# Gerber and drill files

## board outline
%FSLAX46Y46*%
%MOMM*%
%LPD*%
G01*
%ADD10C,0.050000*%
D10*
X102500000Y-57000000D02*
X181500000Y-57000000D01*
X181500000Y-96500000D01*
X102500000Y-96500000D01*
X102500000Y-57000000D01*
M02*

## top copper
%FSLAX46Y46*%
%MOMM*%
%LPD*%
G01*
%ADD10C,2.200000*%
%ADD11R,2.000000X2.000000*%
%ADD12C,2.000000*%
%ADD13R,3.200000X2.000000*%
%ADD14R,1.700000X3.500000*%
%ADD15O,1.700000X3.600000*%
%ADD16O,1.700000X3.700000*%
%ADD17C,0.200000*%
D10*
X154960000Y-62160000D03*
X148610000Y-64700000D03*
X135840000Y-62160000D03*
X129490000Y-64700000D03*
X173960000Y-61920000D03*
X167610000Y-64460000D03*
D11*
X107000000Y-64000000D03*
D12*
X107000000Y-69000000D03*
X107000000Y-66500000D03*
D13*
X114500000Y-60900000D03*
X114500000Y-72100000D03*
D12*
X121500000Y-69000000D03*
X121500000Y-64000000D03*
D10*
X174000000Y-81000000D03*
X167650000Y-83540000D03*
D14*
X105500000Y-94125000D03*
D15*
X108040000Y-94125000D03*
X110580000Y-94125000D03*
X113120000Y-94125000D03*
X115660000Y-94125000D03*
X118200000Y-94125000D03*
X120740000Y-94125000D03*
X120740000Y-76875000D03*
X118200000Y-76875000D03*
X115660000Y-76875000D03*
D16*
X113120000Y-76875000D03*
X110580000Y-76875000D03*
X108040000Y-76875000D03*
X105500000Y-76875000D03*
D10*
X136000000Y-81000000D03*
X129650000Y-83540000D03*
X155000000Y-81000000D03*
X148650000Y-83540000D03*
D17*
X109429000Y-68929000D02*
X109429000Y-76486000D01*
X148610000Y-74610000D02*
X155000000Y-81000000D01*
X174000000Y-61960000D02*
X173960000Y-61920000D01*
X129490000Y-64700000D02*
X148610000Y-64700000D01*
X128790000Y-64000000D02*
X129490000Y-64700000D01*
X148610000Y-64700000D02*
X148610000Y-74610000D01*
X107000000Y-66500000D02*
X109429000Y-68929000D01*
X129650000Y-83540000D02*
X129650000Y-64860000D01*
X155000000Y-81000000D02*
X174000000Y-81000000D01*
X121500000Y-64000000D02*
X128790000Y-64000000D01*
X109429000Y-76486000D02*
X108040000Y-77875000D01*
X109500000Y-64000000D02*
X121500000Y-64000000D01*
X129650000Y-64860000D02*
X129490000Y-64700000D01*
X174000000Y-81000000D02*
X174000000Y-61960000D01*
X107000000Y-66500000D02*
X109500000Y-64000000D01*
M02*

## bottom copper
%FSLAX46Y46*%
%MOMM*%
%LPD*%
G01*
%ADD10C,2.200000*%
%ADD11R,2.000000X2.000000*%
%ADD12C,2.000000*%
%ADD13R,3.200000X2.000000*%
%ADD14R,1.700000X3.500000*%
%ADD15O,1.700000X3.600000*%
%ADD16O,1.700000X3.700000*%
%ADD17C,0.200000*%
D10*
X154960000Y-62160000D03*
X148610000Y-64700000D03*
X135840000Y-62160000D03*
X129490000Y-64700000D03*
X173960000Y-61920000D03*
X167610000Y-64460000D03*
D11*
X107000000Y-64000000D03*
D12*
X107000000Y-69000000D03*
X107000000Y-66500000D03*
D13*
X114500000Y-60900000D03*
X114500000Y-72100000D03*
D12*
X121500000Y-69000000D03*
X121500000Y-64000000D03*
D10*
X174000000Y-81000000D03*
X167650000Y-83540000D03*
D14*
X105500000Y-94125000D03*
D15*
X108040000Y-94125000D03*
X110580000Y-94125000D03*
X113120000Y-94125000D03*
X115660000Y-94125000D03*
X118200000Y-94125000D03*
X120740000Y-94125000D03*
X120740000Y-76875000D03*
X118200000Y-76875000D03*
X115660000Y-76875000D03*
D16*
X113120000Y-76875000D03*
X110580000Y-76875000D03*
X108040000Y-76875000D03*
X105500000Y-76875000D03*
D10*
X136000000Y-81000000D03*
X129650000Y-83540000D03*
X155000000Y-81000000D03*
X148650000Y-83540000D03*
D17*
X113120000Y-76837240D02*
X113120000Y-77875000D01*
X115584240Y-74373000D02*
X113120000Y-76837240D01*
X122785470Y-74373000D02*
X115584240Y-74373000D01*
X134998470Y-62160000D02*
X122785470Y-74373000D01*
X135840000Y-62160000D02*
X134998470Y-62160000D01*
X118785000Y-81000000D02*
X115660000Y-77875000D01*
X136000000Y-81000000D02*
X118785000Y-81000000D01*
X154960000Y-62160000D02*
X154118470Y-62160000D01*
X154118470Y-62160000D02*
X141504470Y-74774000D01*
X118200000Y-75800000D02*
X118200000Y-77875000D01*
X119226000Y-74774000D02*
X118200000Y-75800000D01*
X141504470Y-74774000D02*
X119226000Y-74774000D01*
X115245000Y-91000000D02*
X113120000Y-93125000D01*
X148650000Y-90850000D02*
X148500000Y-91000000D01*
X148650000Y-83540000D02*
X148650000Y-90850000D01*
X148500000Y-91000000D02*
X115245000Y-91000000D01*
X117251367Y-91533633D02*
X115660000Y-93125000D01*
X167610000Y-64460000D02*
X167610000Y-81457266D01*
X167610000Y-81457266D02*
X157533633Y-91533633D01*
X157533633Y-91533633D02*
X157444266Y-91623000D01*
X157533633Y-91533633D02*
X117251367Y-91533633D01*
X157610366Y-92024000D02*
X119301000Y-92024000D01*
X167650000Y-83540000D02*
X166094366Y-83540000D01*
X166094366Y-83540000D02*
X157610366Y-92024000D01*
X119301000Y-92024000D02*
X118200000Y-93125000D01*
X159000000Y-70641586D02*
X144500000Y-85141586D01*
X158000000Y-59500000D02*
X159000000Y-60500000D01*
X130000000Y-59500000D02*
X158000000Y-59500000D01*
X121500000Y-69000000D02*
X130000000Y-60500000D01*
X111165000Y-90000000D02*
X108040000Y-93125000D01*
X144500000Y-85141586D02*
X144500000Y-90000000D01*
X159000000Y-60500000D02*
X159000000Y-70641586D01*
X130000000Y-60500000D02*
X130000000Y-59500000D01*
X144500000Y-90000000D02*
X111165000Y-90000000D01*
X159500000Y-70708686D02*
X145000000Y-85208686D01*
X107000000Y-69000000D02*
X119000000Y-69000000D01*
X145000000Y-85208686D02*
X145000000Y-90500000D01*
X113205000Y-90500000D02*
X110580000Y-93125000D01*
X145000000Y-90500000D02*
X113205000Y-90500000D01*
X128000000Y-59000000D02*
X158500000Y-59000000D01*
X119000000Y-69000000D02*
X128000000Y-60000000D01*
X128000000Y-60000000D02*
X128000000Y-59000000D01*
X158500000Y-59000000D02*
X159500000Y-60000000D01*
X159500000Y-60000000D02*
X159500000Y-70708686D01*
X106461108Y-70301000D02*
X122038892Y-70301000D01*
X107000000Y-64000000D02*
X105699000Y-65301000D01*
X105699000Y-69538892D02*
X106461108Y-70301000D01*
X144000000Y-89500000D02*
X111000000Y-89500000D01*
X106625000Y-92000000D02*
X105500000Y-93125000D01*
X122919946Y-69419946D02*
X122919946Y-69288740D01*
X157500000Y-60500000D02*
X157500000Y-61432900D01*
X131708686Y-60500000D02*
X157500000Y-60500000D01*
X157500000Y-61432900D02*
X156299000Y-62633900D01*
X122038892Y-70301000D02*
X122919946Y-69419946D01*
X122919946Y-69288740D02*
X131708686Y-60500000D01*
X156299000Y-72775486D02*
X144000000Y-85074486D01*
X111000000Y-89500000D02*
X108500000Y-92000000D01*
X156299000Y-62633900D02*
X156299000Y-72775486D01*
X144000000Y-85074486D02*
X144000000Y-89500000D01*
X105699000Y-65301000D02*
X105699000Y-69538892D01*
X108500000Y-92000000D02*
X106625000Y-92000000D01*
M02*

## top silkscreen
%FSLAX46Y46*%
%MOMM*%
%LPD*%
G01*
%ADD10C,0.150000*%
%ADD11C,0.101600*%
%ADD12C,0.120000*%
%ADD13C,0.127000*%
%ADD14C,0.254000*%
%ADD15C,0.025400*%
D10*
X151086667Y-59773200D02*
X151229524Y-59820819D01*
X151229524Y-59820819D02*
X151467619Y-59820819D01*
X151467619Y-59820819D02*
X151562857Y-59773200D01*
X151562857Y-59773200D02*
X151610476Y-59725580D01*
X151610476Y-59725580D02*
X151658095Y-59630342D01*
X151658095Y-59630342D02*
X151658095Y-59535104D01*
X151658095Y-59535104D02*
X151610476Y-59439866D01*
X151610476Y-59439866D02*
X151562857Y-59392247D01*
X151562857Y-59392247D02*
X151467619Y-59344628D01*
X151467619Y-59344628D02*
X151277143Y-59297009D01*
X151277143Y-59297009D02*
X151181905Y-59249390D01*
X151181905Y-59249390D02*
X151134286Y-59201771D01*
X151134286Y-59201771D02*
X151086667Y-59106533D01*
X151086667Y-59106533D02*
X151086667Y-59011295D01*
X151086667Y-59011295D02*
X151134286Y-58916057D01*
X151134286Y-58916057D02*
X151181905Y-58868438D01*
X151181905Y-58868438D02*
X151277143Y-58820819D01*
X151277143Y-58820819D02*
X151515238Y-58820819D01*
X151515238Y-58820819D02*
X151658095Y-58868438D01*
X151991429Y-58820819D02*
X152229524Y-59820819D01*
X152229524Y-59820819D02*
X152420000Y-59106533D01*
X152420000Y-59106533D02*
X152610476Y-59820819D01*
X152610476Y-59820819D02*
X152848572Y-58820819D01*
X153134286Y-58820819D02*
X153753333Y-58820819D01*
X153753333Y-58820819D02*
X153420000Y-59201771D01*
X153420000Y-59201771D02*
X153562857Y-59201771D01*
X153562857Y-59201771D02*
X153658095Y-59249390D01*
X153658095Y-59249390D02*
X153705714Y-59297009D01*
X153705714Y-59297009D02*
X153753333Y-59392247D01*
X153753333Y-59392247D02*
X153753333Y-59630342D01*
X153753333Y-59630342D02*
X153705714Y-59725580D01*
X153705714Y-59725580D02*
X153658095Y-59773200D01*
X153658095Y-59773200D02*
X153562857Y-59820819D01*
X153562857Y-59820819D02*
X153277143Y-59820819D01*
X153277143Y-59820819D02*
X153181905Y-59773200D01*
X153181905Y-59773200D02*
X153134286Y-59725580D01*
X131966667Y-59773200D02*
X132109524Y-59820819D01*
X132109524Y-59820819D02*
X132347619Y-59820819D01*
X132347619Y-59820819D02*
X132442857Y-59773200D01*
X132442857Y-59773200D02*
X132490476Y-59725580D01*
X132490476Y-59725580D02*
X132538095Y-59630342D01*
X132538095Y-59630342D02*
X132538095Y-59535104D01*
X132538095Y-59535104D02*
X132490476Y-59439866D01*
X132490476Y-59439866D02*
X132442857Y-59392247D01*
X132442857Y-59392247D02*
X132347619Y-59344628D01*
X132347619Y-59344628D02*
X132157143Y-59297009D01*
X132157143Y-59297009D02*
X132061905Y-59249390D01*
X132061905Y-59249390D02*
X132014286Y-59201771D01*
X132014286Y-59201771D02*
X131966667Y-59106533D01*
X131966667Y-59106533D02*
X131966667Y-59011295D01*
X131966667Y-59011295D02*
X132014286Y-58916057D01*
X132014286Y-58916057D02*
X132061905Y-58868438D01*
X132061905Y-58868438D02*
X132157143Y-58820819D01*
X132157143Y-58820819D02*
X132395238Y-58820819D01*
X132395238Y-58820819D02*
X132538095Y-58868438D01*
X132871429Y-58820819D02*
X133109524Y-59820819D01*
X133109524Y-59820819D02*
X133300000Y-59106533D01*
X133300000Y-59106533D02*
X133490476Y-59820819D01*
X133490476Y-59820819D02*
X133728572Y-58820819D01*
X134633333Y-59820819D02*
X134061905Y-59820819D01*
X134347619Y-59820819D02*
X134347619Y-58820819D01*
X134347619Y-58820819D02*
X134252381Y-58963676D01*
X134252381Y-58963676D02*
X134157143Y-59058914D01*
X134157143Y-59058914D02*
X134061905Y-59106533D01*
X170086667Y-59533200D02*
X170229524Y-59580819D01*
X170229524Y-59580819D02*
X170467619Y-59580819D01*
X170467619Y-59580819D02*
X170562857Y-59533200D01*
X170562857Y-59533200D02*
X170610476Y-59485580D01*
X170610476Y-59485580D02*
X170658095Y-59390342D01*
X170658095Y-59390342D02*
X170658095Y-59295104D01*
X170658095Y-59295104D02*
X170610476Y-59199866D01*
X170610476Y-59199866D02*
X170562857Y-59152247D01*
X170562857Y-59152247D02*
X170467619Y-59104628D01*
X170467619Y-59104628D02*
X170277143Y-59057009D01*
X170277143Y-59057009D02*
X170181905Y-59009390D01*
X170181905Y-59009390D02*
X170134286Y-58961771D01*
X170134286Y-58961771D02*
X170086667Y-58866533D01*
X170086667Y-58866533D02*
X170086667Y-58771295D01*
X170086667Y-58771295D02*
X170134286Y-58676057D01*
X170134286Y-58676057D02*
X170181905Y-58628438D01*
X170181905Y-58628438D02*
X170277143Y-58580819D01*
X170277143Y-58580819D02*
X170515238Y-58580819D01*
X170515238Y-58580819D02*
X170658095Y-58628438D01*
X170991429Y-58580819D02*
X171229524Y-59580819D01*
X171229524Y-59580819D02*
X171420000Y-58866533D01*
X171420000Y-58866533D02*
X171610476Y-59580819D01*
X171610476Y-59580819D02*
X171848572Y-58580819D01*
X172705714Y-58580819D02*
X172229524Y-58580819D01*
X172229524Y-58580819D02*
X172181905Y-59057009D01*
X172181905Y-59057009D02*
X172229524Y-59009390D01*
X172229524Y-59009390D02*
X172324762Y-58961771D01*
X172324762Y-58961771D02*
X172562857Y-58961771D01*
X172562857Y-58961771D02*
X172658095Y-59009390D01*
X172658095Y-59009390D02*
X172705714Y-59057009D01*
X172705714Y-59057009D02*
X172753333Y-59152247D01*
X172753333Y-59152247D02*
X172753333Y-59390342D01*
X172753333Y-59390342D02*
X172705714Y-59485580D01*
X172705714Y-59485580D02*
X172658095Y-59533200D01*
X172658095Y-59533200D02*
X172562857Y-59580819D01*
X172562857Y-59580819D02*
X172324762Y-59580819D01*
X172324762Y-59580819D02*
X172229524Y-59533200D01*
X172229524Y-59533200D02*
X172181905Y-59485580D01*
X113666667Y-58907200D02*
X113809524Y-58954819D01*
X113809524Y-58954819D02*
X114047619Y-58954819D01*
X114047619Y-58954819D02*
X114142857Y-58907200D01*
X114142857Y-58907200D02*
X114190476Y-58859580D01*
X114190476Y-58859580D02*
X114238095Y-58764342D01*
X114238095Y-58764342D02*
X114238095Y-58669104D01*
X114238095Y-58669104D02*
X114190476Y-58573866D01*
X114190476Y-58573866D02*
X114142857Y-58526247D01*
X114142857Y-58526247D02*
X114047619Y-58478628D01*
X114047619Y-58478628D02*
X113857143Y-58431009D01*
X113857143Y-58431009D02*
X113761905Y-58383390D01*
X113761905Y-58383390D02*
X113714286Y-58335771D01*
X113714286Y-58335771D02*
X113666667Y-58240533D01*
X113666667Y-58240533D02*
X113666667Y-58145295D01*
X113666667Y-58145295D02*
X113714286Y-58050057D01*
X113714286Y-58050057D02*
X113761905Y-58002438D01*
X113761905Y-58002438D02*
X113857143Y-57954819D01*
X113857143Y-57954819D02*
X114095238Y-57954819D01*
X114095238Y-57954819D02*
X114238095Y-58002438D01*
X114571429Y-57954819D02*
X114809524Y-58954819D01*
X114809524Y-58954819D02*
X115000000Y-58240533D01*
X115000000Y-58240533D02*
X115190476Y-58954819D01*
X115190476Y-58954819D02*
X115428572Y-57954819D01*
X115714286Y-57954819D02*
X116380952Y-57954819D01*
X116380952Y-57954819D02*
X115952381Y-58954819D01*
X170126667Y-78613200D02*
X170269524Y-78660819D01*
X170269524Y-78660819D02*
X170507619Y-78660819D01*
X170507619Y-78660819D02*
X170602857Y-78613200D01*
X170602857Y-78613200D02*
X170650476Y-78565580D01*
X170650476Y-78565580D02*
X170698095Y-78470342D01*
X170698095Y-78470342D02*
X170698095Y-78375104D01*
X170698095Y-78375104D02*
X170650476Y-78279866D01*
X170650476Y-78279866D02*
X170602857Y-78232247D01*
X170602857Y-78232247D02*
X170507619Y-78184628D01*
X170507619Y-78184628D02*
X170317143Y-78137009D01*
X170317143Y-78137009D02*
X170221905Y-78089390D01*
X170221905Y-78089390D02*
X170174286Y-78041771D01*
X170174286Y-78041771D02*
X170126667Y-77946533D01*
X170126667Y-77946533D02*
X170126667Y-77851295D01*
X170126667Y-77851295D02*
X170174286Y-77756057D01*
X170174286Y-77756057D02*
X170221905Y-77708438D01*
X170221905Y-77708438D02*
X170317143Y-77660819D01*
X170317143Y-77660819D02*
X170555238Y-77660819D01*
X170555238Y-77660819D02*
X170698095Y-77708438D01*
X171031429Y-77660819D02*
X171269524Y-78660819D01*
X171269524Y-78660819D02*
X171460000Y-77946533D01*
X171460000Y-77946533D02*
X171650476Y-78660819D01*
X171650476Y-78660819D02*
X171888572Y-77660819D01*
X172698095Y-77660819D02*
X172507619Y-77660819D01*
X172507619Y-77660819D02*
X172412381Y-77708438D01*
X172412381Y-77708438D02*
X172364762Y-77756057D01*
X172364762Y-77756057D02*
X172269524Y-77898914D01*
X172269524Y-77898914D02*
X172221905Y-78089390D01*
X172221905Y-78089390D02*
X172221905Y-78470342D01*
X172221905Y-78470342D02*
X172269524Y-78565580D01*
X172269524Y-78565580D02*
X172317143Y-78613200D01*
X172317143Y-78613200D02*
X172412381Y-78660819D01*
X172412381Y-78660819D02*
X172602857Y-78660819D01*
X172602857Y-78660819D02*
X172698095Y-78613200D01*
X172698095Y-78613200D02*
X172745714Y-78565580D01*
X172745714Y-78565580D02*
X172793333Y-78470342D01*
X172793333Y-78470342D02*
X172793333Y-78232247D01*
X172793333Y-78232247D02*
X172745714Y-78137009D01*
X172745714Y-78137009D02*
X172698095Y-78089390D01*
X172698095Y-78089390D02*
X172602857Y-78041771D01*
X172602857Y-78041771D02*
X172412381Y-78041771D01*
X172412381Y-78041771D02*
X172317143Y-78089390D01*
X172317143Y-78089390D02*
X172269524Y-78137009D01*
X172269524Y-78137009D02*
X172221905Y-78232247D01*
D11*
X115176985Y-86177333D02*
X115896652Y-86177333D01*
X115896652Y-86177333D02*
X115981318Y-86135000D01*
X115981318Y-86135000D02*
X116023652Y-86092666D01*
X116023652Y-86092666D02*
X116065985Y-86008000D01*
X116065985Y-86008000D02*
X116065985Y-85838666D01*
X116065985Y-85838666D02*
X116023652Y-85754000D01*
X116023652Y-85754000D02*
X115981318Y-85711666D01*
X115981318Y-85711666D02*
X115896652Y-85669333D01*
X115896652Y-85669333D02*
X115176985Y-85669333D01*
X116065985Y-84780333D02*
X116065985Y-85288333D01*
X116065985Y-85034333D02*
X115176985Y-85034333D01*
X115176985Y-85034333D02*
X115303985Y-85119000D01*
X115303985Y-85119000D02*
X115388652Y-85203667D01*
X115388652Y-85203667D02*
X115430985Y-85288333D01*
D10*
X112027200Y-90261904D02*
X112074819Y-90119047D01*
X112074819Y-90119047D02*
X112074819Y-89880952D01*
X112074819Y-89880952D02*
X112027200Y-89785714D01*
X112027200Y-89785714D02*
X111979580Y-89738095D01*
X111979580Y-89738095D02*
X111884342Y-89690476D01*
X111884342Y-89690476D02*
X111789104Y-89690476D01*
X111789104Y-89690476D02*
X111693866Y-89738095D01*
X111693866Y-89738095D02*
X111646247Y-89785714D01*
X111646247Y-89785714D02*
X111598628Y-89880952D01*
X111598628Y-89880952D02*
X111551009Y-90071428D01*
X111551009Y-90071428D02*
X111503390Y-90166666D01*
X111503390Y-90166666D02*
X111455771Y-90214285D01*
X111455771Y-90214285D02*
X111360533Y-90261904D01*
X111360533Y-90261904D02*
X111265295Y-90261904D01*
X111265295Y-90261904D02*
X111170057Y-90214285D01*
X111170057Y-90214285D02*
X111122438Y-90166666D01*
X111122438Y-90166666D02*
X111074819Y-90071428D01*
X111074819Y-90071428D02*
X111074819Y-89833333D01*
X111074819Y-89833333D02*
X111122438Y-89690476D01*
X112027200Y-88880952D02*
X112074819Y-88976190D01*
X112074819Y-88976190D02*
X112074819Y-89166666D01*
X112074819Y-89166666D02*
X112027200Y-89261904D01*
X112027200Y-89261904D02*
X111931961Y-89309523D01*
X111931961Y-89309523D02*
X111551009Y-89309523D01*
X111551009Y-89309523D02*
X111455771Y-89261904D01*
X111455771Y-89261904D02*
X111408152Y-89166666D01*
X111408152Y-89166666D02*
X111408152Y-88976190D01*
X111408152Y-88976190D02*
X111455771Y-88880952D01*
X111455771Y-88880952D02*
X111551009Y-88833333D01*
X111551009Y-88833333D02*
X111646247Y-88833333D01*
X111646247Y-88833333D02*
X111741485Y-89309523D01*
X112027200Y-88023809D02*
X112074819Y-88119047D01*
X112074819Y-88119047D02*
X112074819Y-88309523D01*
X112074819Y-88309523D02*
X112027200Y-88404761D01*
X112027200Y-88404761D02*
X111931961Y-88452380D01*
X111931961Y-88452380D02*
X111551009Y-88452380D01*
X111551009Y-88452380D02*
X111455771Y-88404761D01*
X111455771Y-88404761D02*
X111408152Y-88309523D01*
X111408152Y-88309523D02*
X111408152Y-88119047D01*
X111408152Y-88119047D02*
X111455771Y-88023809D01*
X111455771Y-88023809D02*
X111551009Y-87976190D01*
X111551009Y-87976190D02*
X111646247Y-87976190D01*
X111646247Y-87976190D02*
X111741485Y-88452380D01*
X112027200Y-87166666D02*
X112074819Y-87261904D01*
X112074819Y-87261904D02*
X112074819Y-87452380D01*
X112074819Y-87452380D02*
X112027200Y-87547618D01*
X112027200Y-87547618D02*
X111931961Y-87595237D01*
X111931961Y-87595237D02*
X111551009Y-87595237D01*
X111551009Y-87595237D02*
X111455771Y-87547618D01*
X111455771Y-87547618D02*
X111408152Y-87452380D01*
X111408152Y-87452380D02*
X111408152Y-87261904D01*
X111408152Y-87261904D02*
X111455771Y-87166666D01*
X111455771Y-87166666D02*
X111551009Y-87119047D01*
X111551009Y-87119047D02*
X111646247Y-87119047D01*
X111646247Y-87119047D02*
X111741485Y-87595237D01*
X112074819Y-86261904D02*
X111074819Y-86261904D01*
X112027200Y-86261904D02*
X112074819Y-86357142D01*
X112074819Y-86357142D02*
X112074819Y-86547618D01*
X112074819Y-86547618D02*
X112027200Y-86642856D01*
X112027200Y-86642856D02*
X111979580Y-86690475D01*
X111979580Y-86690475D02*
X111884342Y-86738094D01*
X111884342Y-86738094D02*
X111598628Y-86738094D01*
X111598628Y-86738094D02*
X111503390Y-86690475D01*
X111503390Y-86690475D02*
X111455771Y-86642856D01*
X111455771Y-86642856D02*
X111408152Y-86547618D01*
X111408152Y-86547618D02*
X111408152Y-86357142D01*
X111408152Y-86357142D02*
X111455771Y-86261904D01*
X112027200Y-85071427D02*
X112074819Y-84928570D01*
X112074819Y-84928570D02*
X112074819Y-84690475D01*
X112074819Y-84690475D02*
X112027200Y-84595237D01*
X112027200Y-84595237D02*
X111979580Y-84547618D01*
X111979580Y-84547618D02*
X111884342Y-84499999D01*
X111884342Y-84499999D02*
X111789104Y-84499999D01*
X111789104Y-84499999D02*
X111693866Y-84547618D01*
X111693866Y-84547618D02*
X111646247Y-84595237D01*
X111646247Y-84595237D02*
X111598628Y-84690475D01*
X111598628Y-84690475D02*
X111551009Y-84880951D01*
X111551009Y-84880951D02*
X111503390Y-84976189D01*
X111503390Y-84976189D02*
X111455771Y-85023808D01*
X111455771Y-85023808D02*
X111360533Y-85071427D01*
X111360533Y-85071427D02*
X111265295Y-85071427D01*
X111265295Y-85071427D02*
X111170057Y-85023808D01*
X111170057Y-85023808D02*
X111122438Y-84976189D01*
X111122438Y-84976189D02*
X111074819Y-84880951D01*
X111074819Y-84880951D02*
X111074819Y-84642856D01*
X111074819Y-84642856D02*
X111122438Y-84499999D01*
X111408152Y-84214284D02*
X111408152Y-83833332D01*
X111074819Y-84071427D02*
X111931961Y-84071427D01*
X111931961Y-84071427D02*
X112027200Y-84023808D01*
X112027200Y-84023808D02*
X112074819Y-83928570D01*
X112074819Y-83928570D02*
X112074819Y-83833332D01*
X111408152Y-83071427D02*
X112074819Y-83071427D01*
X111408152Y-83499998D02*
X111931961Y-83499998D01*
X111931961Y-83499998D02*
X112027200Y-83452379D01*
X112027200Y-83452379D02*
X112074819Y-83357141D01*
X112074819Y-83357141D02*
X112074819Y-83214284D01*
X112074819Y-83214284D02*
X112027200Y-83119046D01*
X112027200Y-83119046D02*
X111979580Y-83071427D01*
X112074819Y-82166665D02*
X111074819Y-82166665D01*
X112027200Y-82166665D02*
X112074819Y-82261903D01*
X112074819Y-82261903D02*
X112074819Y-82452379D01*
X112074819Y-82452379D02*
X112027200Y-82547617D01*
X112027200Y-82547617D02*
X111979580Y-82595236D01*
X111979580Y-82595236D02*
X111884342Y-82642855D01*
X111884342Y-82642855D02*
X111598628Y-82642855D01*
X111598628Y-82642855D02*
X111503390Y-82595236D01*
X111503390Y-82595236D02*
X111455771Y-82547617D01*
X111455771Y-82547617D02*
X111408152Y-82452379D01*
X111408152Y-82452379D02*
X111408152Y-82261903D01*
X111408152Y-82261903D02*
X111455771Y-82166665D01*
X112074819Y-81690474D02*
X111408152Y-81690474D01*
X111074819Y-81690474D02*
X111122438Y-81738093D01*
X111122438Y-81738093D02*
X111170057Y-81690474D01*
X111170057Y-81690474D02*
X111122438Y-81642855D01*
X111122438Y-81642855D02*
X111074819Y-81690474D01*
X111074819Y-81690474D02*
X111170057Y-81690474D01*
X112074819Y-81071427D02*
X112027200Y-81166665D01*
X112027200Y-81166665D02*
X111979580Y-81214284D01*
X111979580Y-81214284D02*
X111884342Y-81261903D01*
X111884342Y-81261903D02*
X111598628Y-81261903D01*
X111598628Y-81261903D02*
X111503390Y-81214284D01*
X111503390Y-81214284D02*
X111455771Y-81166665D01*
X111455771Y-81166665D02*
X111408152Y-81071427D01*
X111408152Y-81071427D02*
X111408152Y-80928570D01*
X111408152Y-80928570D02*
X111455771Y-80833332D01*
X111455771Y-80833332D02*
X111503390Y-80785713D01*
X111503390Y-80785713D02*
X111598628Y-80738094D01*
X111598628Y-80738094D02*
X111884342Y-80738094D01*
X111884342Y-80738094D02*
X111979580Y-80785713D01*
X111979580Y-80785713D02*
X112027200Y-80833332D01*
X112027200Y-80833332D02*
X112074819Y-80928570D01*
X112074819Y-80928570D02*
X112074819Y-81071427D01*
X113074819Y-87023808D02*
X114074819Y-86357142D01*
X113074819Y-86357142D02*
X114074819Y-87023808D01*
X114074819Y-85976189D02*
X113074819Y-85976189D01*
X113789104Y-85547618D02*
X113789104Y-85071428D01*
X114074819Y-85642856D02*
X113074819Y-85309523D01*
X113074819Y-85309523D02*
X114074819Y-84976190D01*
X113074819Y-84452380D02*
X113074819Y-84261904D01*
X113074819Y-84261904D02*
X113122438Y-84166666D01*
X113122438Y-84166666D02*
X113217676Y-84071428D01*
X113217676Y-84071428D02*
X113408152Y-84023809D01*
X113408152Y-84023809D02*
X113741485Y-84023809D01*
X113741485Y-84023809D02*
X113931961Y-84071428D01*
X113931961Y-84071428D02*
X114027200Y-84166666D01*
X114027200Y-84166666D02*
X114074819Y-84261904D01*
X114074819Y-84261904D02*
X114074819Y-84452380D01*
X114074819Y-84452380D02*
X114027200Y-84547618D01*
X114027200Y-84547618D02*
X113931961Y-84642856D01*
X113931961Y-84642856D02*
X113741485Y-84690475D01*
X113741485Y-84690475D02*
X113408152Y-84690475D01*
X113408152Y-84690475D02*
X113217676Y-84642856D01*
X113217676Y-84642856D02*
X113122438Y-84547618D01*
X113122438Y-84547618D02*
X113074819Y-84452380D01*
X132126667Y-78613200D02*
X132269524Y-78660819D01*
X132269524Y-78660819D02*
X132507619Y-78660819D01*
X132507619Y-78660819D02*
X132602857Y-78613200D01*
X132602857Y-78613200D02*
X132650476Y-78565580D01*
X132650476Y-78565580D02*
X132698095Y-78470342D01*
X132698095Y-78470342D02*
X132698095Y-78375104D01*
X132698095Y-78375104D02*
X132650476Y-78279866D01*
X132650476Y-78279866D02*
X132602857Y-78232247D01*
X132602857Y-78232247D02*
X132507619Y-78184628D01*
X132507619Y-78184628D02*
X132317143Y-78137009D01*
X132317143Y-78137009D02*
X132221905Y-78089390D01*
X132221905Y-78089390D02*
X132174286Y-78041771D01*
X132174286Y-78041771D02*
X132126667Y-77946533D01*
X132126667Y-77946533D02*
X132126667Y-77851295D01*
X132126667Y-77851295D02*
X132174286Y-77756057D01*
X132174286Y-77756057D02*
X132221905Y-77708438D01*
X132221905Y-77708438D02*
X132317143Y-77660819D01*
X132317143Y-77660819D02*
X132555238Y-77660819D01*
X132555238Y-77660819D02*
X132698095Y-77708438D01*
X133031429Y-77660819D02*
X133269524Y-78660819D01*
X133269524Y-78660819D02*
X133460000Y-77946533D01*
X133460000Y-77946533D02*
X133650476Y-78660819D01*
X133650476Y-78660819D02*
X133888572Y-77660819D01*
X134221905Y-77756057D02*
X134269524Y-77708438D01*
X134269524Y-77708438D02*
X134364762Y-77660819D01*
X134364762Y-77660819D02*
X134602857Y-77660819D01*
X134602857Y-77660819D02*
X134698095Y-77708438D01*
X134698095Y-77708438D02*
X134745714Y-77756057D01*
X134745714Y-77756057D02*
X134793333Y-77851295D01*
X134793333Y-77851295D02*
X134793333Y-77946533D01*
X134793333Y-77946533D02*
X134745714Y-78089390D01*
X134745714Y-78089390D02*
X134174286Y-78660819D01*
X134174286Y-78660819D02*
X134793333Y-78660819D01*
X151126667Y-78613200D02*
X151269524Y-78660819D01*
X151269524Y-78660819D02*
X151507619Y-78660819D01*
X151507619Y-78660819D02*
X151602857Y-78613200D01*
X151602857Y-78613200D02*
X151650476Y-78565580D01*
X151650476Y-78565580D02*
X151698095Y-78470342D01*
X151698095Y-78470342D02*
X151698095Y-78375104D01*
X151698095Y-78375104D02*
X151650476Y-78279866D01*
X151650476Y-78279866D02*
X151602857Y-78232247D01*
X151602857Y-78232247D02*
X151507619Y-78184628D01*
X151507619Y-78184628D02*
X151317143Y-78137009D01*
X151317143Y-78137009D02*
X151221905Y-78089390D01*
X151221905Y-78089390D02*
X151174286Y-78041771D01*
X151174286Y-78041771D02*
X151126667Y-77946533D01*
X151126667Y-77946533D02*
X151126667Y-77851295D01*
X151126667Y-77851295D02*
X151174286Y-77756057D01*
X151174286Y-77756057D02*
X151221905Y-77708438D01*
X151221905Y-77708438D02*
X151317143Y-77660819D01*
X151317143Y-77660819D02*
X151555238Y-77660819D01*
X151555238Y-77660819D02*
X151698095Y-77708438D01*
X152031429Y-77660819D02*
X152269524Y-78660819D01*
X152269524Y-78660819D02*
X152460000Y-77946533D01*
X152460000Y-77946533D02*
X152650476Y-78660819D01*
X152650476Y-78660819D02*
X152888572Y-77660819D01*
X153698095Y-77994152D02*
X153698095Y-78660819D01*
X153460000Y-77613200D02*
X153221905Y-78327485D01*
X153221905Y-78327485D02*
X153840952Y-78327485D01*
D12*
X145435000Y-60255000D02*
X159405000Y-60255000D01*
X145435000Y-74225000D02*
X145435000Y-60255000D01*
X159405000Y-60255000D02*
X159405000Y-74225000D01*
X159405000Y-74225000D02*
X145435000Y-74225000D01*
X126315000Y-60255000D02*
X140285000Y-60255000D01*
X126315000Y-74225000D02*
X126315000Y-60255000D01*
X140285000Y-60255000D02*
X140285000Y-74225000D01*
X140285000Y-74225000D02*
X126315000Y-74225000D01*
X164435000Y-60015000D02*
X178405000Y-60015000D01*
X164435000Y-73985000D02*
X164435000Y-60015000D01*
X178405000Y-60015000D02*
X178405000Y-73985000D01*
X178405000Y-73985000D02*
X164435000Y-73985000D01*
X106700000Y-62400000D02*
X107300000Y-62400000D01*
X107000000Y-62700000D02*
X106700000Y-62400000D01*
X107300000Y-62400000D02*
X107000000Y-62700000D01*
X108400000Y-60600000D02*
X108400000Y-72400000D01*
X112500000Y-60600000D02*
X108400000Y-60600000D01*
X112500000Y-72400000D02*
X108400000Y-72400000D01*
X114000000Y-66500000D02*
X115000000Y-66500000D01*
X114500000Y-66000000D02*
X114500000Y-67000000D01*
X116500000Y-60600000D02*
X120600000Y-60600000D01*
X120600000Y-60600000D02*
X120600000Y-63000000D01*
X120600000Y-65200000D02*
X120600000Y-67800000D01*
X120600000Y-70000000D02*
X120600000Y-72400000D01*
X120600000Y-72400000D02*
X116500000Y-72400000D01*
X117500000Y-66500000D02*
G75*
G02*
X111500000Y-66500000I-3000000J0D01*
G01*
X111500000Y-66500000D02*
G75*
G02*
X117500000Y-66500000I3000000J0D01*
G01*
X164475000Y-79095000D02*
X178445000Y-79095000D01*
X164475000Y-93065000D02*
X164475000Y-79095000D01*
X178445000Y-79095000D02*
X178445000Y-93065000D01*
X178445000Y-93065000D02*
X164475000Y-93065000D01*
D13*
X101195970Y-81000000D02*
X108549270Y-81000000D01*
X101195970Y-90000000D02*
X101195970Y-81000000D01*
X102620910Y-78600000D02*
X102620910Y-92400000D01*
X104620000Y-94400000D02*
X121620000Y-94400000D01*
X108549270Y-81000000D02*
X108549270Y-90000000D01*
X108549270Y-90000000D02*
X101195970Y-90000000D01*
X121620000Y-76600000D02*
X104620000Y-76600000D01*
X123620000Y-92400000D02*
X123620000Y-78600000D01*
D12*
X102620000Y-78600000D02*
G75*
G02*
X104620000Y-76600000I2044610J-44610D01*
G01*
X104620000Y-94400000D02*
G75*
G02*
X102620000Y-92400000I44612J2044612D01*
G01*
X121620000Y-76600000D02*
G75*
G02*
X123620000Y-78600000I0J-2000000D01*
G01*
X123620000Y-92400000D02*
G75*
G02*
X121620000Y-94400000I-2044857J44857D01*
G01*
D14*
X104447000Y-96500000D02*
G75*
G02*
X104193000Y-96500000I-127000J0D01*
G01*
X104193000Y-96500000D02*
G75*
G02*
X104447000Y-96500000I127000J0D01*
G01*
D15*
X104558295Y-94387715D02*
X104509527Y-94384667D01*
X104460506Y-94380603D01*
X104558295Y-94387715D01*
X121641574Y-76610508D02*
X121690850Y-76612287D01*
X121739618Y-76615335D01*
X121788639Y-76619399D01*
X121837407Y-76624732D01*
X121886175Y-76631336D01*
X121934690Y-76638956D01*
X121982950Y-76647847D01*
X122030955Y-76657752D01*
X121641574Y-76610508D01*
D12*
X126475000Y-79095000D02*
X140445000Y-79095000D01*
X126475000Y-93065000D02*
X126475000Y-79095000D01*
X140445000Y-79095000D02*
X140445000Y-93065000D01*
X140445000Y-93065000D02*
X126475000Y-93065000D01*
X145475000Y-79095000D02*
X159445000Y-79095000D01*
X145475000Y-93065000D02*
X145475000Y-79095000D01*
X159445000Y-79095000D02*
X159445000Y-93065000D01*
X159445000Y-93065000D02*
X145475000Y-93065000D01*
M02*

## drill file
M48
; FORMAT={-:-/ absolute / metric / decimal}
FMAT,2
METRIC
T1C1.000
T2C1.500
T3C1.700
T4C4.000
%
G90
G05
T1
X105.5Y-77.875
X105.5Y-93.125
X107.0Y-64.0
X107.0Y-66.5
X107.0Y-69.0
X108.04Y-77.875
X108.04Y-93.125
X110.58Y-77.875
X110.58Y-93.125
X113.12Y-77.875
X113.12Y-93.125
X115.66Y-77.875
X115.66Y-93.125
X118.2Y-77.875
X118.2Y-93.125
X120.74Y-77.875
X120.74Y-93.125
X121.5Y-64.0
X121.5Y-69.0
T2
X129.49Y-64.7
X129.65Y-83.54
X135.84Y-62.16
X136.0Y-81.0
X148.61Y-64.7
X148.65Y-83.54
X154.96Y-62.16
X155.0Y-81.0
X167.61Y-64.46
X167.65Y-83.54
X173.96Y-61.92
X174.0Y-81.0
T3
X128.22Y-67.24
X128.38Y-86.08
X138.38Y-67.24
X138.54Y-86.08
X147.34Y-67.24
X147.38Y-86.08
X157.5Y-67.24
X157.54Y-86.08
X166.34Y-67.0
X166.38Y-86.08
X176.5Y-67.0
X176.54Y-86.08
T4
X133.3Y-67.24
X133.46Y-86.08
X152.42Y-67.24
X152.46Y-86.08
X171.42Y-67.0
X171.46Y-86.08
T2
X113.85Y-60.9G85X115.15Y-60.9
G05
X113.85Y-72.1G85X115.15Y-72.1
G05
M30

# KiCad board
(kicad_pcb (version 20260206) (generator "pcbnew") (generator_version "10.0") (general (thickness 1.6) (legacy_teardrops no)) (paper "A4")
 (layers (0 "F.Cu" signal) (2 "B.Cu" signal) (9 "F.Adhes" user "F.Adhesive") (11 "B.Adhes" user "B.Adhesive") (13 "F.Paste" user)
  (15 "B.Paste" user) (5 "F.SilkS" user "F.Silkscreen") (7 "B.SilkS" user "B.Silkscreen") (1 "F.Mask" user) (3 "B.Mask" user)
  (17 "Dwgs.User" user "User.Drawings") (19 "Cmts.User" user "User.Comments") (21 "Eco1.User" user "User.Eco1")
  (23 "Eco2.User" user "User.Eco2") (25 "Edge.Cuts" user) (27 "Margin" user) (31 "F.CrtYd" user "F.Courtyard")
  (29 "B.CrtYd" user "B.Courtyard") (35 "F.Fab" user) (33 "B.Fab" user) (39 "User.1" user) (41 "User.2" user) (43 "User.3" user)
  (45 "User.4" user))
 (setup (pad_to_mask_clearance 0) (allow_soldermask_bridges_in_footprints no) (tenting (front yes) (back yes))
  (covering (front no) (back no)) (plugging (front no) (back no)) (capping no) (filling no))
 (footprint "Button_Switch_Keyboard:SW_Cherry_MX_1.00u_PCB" (layer "F.Cu") (at 154.96 62.16)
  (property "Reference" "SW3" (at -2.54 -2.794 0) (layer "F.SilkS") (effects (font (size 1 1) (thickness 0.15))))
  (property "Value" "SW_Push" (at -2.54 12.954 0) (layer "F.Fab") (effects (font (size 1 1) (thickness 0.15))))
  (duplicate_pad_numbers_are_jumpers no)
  (fp_line (start -9.525 -1.905) (end 4.445 -1.905) (stroke (width 0.12) (type solid)) (layer "F.SilkS"))
  (fp_line (start -9.525 12.065) (end -9.525 -1.905) (stroke (width 0.12) (type solid)) (layer "F.SilkS"))
  (fp_line (start 4.445 -1.905) (end 4.445 12.065) (stroke (width 0.12) (type solid)) (layer "F.SilkS"))
  (fp_line (start 4.445 12.065) (end -9.525 12.065) (stroke (width 0.12) (type solid)) (layer "F.SilkS"))
  (pad "" np_thru_hole circle (at -7.62 5.08) (size 1.7 1.7) (drill 1.7) (layers "*.Cu" "*.Mask"))
  (pad "" np_thru_hole circle (at -2.54 5.08) (size 4 4) (drill 4) (layers "*.Cu" "*.Mask"))
  (pad "" np_thru_hole circle (at 2.54 5.08) (size 1.7 1.7) (drill 1.7) (layers "*.Cu" "*.Mask"))
  (pad "1" thru_hole circle (at 0 0) (size 2.2 2.2) (drill 1.5) (layers "*.Cu" "*.Mask") (remove_unused_layers no)
   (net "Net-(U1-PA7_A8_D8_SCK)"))
  (pad "2" thru_hole circle (at -6.35 2.54) (size 2.2 2.2) (drill 1.5) (layers "*.Cu" "*.Mask") (remove_unused_layers no) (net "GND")))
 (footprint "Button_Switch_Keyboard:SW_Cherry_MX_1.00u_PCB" (layer "F.Cu") (at 135.84 62.16)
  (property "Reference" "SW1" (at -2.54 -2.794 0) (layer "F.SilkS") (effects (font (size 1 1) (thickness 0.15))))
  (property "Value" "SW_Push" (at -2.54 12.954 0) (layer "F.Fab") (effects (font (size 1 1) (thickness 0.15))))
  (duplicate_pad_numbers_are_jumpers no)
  (fp_line (start -9.525 -1.905) (end 4.445 -1.905) (stroke (width 0.12) (type solid)) (layer "F.SilkS"))
  (fp_line (start -9.525 12.065) (end -9.525 -1.905) (stroke (width 0.12) (type solid)) (layer "F.SilkS"))
  (fp_line (start 4.445 -1.905) (end 4.445 12.065) (stroke (width 0.12) (type solid)) (layer "F.SilkS"))
  (fp_line (start 4.445 12.065) (end -9.525 12.065) (stroke (width 0.12) (type solid)) (layer "F.SilkS"))
  (pad "" np_thru_hole circle (at -7.62 5.08) (size 1.7 1.7) (drill 1.7) (layers "*.Cu" "*.Mask"))
  (pad "" np_thru_hole circle (at -2.54 5.08) (size 4 4) (drill 4) (layers "*.Cu" "*.Mask"))
  (pad "" np_thru_hole circle (at 2.54 5.08) (size 1.7 1.7) (drill 1.7) (layers "*.Cu" "*.Mask"))
  (pad "1" thru_hole circle (at 0 0) (size 2.2 2.2) (drill 1.5) (layers "*.Cu" "*.Mask") (remove_unused_layers no)
   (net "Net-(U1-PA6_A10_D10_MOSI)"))
  (pad "2" thru_hole circle (at -6.35 2.54) (size 2.2 2.2) (drill 1.5) (layers "*.Cu" "*.Mask") (remove_unused_layers no) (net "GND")))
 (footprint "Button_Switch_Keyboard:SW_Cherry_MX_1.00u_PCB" (layer "F.Cu") (at 173.96 61.92)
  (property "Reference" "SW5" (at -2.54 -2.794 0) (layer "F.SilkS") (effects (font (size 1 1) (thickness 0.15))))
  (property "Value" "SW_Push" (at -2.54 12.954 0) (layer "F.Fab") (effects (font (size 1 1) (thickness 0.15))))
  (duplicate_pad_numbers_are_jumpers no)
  (fp_line (start -9.525 -1.905) (end 4.445 -1.905) (stroke (width 0.12) (type solid)) (layer "F.SilkS"))
  (fp_line (start -9.525 12.065) (end -9.525 -1.905) (stroke (width 0.12) (type solid)) (layer "F.SilkS"))
  (fp_line (start 4.445 -1.905) (end 4.445 12.065) (stroke (width 0.12) (type solid)) (layer "F.SilkS"))
  (fp_line (start 4.445 12.065) (end -9.525 12.065) (stroke (width 0.12) (type solid)) (layer "F.SilkS"))
  (pad "" np_thru_hole circle (at -7.62 5.08) (size 1.7 1.7) (drill 1.7) (layers "*.Cu" "*.Mask"))
  (pad "" np_thru_hole circle (at -2.54 5.08) (size 4 4) (drill 4) (layers "*.Cu" "*.Mask"))
  (pad "" np_thru_hole circle (at 2.54 5.08) (size 1.7 1.7) (drill 1.7) (layers "*.Cu" "*.Mask"))
  (pad "1" thru_hole circle (at 0 0) (size 2.2 2.2) (drill 1.5) (layers "*.Cu" "*.Mask") (remove_unused_layers no) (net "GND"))
  (pad "2" thru_hole circle (at -6.35 2.54) (size 2.2 2.2) (drill 1.5) (layers "*.Cu" "*.Mask") (remove_unused_layers no)
   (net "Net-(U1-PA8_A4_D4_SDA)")))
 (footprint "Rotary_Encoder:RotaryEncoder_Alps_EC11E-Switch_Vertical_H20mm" (layer "F.Cu") (at 107 64)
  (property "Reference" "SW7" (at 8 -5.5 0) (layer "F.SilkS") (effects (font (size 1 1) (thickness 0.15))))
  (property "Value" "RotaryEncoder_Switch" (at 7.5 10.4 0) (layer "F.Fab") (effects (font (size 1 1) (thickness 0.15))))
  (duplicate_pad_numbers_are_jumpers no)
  (fp_line (start -0.3 -1.6) (end 0.3 -1.6) (stroke (width 0.12) (type solid)) (layer "F.SilkS"))
  (fp_line (start 0 -1.3) (end -0.3 -1.6) (stroke (width 0.12) (type solid)) (layer "F.SilkS"))
  (fp_line (start 0.3 -1.6) (end 0 -1.3) (stroke (width 0.12) (type solid)) (layer "F.SilkS"))
  (fp_line (start 1.4 -3.4) (end 1.4 8.4) (stroke (width 0.12) (type solid)) (layer "F.SilkS"))
  (fp_line (start 5.5 -3.4) (end 1.4 -3.4) (stroke (width 0.12) (type solid)) (layer "F.SilkS"))
  (fp_line (start 5.5 8.4) (end 1.4 8.4) (stroke (width 0.12) (type solid)) (layer "F.SilkS"))
  (fp_line (start 7 2.5) (end 8 2.5) (stroke (width 0.12) (type solid)) (layer "F.SilkS"))
  (fp_line (start 7.5 2) (end 7.5 3) (stroke (width 0.12) (type solid)) (layer "F.SilkS"))
  (fp_line (start 9.5 -3.4) (end 13.6 -3.4) (stroke (width 0.12) (type solid)) (layer "F.SilkS"))
  (fp_line (start 13.6 -3.4) (end 13.6 -1) (stroke (width 0.12) (type solid)) (layer "F.SilkS"))
  (fp_line (start 13.6 1.2) (end 13.6 3.8) (stroke (width 0.12) (type solid)) (layer "F.SilkS"))
  (fp_line (start 13.6 6) (end 13.6 8.4) (stroke (width 0.12) (type solid)) (layer "F.SilkS"))
  (fp_line (start 13.6 8.4) (end 9.5 8.4) (stroke (width 0.12) (type solid)) (layer "F.SilkS"))
  (fp_circle (center 7.5 2.5) (end 10.5 2.5) (stroke (width 0.12) (type solid)) (fill no) (layer "F.SilkS"))
  (pad "A" thru_hole rect (at 0 0) (size 2 2) (drill 1) (layers "*.Cu" "*.Mask") (remove_unused_layers no) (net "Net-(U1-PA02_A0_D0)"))
  (pad "B" thru_hole circle (at 0 5) (size 2 2) (drill 1) (layers "*.Cu" "*.Mask") (remove_unused_layers no) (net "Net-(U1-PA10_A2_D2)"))
  (pad "C" thru_hole circle (at 0 2.5) (size 2 2) (drill 1) (layers "*.Cu" "*.Mask") (remove_unused_layers no) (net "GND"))
  (pad "MP" thru_hole rect (at 7.5 -3.1) (size 3.2 2) (drill oval 2.8 1.5) (layers "*.Cu" "*.Mask") (remove_unused_layers no))
  (pad "MP" thru_hole rect (at 7.5 8.1) (size 3.2 2) (drill oval 2.8 1.5) (layers "*.Cu" "*.Mask") (remove_unused_layers no))
  (pad "S1" thru_hole circle (at 14.5 5) (size 2 2) (drill 1) (layers "*.Cu" "*.Mask") (remove_unused_layers no) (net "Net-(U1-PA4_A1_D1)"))
  (pad "S2" thru_hole circle (at 14.5 0) (size 2 2) (drill 1) (layers "*.Cu" "*.Mask") (remove_unused_layers no) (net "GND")))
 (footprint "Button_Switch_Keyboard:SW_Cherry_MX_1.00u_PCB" (layer "F.Cu") (at 174 81)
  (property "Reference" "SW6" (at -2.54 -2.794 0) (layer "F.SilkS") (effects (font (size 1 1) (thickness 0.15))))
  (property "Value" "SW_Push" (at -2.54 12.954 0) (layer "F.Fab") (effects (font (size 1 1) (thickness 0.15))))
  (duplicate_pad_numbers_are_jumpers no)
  (fp_line (start -9.525 -1.905) (end 4.445 -1.905) (stroke (width 0.12) (type solid)) (layer "F.SilkS"))
  (fp_line (start -9.525 12.065) (end -9.525 -1.905) (stroke (width 0.12) (type solid)) (layer "F.SilkS"))
  (fp_line (start 4.445 -1.905) (end 4.445 12.065) (stroke (width 0.12) (type solid)) (layer "F.SilkS"))
  (fp_line (start 4.445 12.065) (end -9.525 12.065) (stroke (width 0.12) (type solid)) (layer "F.SilkS"))
  (pad "" np_thru_hole circle (at -7.62 5.08) (size 1.7 1.7) (drill 1.7) (layers "*.Cu" "*.Mask"))
  (pad "" np_thru_hole circle (at -2.54 5.08) (size 4 4) (drill 4) (layers "*.Cu" "*.Mask"))
  (pad "" np_thru_hole circle (at 2.54 5.08) (size 1.7 1.7) (drill 1.7) (layers "*.Cu" "*.Mask"))
  (pad "1" thru_hole circle (at 0 0) (size 2.2 2.2) (drill 1.5) (layers "*.Cu" "*.Mask") (remove_unused_layers no) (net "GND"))
  (pad "2" thru_hole circle (at -6.35 2.54) (size 2.2 2.2) (drill 1.5) (layers "*.Cu" "*.Mask") (remove_unused_layers no)
   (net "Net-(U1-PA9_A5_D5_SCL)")))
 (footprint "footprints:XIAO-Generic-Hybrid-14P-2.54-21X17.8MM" (layer "F.Cu") (at 113.12 85.5 90)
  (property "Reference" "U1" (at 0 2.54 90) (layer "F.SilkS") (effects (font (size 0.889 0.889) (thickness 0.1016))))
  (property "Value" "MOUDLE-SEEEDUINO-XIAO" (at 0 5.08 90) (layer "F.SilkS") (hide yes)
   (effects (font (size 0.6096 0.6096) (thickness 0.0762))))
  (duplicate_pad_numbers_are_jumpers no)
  (fp_line (start 4.5 -11.92403) (end 4.5 -4.57073) (stroke (width 0.127) (type solid)) (layer "F.SilkS"))
  (fp_line (start -4.5 -11.92403) (end 4.5 -11.92403) (stroke (width 0.127) (type solid)) (layer "F.SilkS"))
  (fp_line (start 6.9 -10.49909) (end -6.9 -10.49909) (stroke (width 0.127) (type solid)) (layer "F.SilkS"))
  (fp_line (start -8.9 -8.5) (end -8.9 8.5) (stroke (width 0.127) (type solid)) (layer "F.SilkS"))
  (fp_line (start 4.5 -4.57073) (end -4.5 -4.57073) (stroke (width 0.127) (type solid)) (layer "F.SilkS"))
  (fp_line (start -4.5 -4.57073) (end -4.5 -11.92403) (stroke (width 0.127) (type solid)) (layer "F.SilkS"))
  (fp_line (start 8.9 8.5) (end 8.9 -8.5) (stroke (width 0.127) (type solid)) (layer "F.SilkS"))
  (fp_line (start -6.9 10.5) (end 6.9 10.5) (stroke (width 0.127) (type solid)) (layer "F.SilkS"))
  (fp_arc (start 6.9 -10.5) (mid 8.301491 -9.901491) (end 8.9 -8.5) (stroke (width 0.12) (type solid)) (layer "F.SilkS"))
  (fp_arc (start -8.9 -8.5) (mid -8.301491 -9.901491) (end -6.9 -10.5) (stroke (width 0.12) (type solid)) (layer "F.SilkS"))
  (fp_arc (start 8.9 8.5) (mid 8.314214 9.914214) (end 6.9 10.5) (stroke (width 0.12) (type solid)) (layer "F.SilkS"))
  (fp_arc (start -6.9 10.5) (mid -8.301423 9.901423) (end -8.9 8.5) (stroke (width 0.12) (type solid)) (layer "F.SilkS"))
  (fp_circle (center -11 -8.8) (end -11 -9.054) (stroke (width 0) (type solid)) (fill yes) (layer "F.SilkS"))
  (fp_poly
   (pts (xy -8.887715 -8.561705) (xy -8.884667 -8.610473) (xy -8.880603 -8.659494)) (stroke (width 0.0254) (type solid)) (fill no)
   (layer "F.SilkS"))
  (fp_poly
   (pts (xy 8.889492 8.521574) (xy 8.887713 8.57085) (xy 8.884665 8.619618) (xy 8.880601 8.668639) (xy 8.875268 8.717407)
    (xy 8.868664 8.766175) (xy 8.861044 8.81469) (xy 8.852153 8.86295) (xy 8.842248 8.910955))
   (stroke (width 0.0254) (type solid)) (fill no) (layer "F.SilkS"))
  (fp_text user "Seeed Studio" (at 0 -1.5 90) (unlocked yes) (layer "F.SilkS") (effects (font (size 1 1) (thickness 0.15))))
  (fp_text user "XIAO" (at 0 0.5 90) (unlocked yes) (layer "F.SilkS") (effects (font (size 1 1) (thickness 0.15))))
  (pad "1" thru_hole rect (at -7.625 -7.62 90) (size 3.5 1.7) (drill 1 (offset -1 0)) (layers "*.Cu" "*.Mask") (remove_unused_layers no)
   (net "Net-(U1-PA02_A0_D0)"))
  (pad "2" thru_hole oval (at -7.625 -5.08 90) (size 3.6 1.7) (drill 1 (offset -1 0)) (layers "*.Cu" "*.Mask") (remove_unused_layers no)
   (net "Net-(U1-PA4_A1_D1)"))
  (pad "3" thru_hole oval (at -7.625 -2.54 90) (size 3.6 1.7) (drill 1 (offset -1 0)) (layers "*.Cu" "*.Mask") (remove_unused_layers no)
   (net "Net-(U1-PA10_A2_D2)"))
  (pad "4" thru_hole oval (at -7.625 0 90) (size 3.6 1.7) (drill 1 (offset -1 0)) (layers "*.Cu" "*.Mask") (remove_unused_layers no)
   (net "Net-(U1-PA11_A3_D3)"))
  (pad "5" thru_hole oval (at -7.625 2.54 90) (size 3.6 1.7) (drill 1 (offset -1 0)) (layers "*.Cu" "*.Mask") (remove_unused_layers no)
   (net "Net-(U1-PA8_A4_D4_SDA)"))
  (pad "6" thru_hole oval (at -7.625 5.08 270) (size 3.6 1.7) (drill 1 (offset 1 0)) (layers "*.Cu" "*.Mask") (remove_unused_layers no)
   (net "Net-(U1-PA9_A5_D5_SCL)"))
  (pad "7" thru_hole oval (at -7.625 7.62 90) (size 3.6 1.7) (drill 1 (offset -1 0)) (layers "*.Cu" "*.Mask") (remove_unused_layers no)
   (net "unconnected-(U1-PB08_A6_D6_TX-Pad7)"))
  (pad "8" thru_hole oval (at 7.625 7.62 90) (size 3.6 1.7) (drill 1 (offset 1 0)) (layers "*.Cu" "*.Mask") (remove_unused_layers no)
   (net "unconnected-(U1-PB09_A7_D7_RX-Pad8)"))
  (pad "9" thru_hole oval (at 7.625 5.08 90) (size 3.6 1.7) (drill 1 (offset 1 0)) (layers "*.Cu" "*.Mask") (remove_unused_layers no)
   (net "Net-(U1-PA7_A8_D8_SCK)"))
  (pad "10" thru_hole oval (at 7.625 2.54 90) (size 3.6 1.7) (drill 1 (offset 1 0)) (layers "*.Cu" "*.Mask") (remove_unused_layers no)
   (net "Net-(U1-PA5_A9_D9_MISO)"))
  (pad "11" thru_hole oval (at 7.625 0 90) (size 3.7 1.7) (drill 1 (offset 1 0)) (layers "*.Cu" "*.Mask") (remove_unused_layers no)
   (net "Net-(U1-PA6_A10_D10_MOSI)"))
  (pad "12" thru_hole oval (at 7.625 -2.54 90) (size 3.7 1.7) (drill 1 (offset 1 0)) (layers "*.Cu" "*.Mask") (remove_unused_layers no)
   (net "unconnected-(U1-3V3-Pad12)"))
  (pad "13" thru_hole oval (at 7.625 -5.08 90) (size 3.7 1.7) (drill 1 (offset 1 0)) (layers "*.Cu" "*.Mask") (remove_unused_layers no)
   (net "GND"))
  (pad "14" thru_hole oval (at 7.625 -7.62 90) (size 3.7 1.7) (drill 1 (offset 1 0)) (layers "*.Cu" "*.Mask") (remove_unused_layers no)
   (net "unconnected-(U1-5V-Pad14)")))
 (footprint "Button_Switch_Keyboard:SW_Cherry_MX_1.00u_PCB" (layer "F.Cu") (at 136 81)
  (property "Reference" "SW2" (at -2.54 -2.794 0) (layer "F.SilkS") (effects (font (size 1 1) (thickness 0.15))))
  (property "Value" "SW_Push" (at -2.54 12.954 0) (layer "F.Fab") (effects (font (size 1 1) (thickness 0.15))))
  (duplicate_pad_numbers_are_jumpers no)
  (fp_line (start -9.525 -1.905) (end 4.445 -1.905) (stroke (width 0.12) (type solid)) (layer "F.SilkS"))
  (fp_line (start -9.525 12.065) (end -9.525 -1.905) (stroke (width 0.12) (type solid)) (layer "F.SilkS"))
  (fp_line (start 4.445 -1.905) (end 4.445 12.065) (stroke (width 0.12) (type solid)) (layer "F.SilkS"))
  (fp_line (start 4.445 12.065) (end -9.525 12.065) (stroke (width 0.12) (type solid)) (layer "F.SilkS"))
  (pad "" np_thru_hole circle (at -7.62 5.08) (size 1.7 1.7) (drill 1.7) (layers "*.Cu" "*.Mask"))
  (pad "" np_thru_hole circle (at -2.54 5.08) (size 4 4) (drill 4) (layers "*.Cu" "*.Mask"))
  (pad "" np_thru_hole circle (at 2.54 5.08) (size 1.7 1.7) (drill 1.7) (layers "*.Cu" "*.Mask"))
  (pad "1" thru_hole circle (at 0 0) (size 2.2 2.2) (drill 1.5) (layers "*.Cu" "*.Mask") (remove_unused_layers no)
   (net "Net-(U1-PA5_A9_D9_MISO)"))
  (pad "2" thru_hole circle (at -6.35 2.54) (size 2.2 2.2) (drill 1.5) (layers "*.Cu" "*.Mask") (remove_unused_layers no) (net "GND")))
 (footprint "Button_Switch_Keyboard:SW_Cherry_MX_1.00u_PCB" (layer "F.Cu") (at 155 81)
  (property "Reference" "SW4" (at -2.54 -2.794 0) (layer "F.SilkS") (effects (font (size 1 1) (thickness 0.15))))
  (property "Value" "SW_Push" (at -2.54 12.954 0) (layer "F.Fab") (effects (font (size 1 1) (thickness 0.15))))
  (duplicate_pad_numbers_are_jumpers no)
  (fp_line (start -9.525 -1.905) (end 4.445 -1.905) (stroke (width 0.12) (type solid)) (layer "F.SilkS"))
  (fp_line (start -9.525 12.065) (end -9.525 -1.905) (stroke (width 0.12) (type solid)) (layer "F.SilkS"))
  (fp_line (start 4.445 -1.905) (end 4.445 12.065) (stroke (width 0.12) (type solid)) (layer "F.SilkS"))
  (fp_line (start 4.445 12.065) (end -9.525 12.065) (stroke (width 0.12) (type solid)) (layer "F.SilkS"))
  (pad "" np_thru_hole circle (at -7.62 5.08) (size 1.7 1.7) (drill 1.7) (layers "*.Cu" "*.Mask"))
  (pad "" np_thru_hole circle (at -2.54 5.08) (size 4 4) (drill 4) (layers "*.Cu" "*.Mask"))
  (pad "" np_thru_hole circle (at 2.54 5.08) (size 1.7 1.7) (drill 1.7) (layers "*.Cu" "*.Mask"))
  (pad "1" thru_hole circle (at 0 0) (size 2.2 2.2) (drill 1.5) (layers "*.Cu" "*.Mask") (remove_unused_layers no) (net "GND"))
  (pad "2" thru_hole circle (at -6.35 2.54) (size 2.2 2.2) (drill 1.5) (layers "*.Cu" "*.Mask") (remove_unused_layers no)
   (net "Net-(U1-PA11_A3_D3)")))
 (gr_rect (start 102.5 57) (end 181.5 96.5) (stroke (width 0.05) (type default)) (fill no) (layer "Edge.Cuts"))
 (segment (start 113.12 76.83724) (end 113.12 77.875) (width 0.2) (layer "B.Cu") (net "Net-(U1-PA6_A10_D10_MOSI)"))
 (segment (start 115.58424 74.373) (end 113.12 76.83724) (width 0.2) (layer "B.Cu") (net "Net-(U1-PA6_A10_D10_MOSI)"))
 (segment (start 122.78547 74.373) (end 115.58424 74.373) (width 0.2) (layer "B.Cu") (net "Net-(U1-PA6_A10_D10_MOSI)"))
 (segment (start 134.99847 62.16) (end 122.78547 74.373) (width 0.2) (layer "B.Cu") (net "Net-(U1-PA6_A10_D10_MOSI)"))
 (segment (start 135.84 62.16) (end 134.99847 62.16) (width 0.2) (layer "B.Cu") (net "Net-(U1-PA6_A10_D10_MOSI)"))
 (segment (start 109.429 68.929) (end 109.429 76.486) (width 0.2) (layer "F.Cu") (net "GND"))
 (segment (start 148.61 74.61) (end 155 81) (width 0.2) (layer "F.Cu") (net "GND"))
 (segment (start 174 61.96) (end 173.96 61.92) (width 0.2) (layer "F.Cu") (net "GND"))
 (segment (start 129.49 64.7) (end 148.61 64.7) (width 0.2) (layer "F.Cu") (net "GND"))
 (segment (start 128.79 64) (end 129.49 64.7) (width 0.2) (layer "F.Cu") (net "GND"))
 (segment (start 148.61 64.7) (end 148.61 74.61) (width 0.2) (layer "F.Cu") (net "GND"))
 (segment (start 107 66.5) (end 109.429 68.929) (width 0.2) (layer "F.Cu") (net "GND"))
 (segment (start 129.65 83.54) (end 129.65 64.86) (width 0.2) (layer "F.Cu") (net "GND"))
 (segment (start 155 81) (end 174 81) (width 0.2) (layer "F.Cu") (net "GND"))
 (segment (start 121.5 64) (end 128.79 64) (width 0.2) (layer "F.Cu") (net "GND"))
 (segment (start 109.429 76.486) (end 108.04 77.875) (width 0.2) (layer "F.Cu") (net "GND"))
 (segment (start 109.5 64) (end 121.5 64) (width 0.2) (layer "F.Cu") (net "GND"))
 (segment (start 129.65 64.86) (end 129.49 64.7) (width 0.2) (layer "F.Cu") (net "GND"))
 (segment (start 174 81) (end 174 61.96) (width 0.2) (layer "F.Cu") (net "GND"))
 (segment (start 107 66.5) (end 109.5 64) (width 0.2) (layer "F.Cu") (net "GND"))
 (segment (start 118.785 81) (end 115.66 77.875) (width 0.2) (layer "B.Cu") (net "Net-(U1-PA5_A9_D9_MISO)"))
 (segment (start 136 81) (end 118.785 81) (width 0.2) (layer "B.Cu") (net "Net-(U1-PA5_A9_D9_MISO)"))
 (segment (start 154.96 62.16) (end 154.11847 62.16) (width 0.2) (layer "B.Cu") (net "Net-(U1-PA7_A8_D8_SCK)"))
 (segment (start 154.11847 62.16) (end 141.50447 74.774) (width 0.2) (layer "B.Cu") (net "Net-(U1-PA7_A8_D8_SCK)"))
 (segment (start 118.2 75.8) (end 118.2 77.875) (width 0.2) (layer "B.Cu") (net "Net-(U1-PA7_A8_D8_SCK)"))
 (segment (start 119.226 74.774) (end 118.2 75.8) (width 0.2) (layer "B.Cu") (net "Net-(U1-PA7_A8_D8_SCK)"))
 (segment (start 141.50447 74.774) (end 119.226 74.774) (width 0.2) (layer "B.Cu") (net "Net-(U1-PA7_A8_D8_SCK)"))
 (segment (start 115.245 91) (end 113.12 93.125) (width 0.2) (layer "B.Cu") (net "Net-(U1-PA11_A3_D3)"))
 (segment (start 148.65 90.85) (end 148.5 91) (width 0.2) (layer "B.Cu") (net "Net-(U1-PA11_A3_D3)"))
 (segment (start 148.65 83.54) (end 148.65 90.85) (width 0.2) (layer "B.Cu") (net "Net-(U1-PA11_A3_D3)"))
 (segment (start 148.5 91) (end 115.245 91) (width 0.2) (layer "B.Cu") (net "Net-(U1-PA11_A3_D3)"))
 (segment (start 117.251367 91.533633) (end 115.66 93.125) (width 0.2) (layer "B.Cu") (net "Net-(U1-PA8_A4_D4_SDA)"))
 (segment (start 167.61 64.46) (end 167.61 81.457266) (width 0.2) (layer "B.Cu") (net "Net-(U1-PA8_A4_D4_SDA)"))
 (segment (start 167.61 81.457266) (end 157.533633 91.533633) (width 0.2) (layer "B.Cu") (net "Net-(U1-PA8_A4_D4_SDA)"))
 (segment (start 157.533633 91.533633) (end 157.444266 91.623) (width 0.2) (layer "B.Cu") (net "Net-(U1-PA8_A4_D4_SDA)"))
 (segment (start 157.533633 91.533633) (end 117.251367 91.533633) (width 0.2) (layer "B.Cu") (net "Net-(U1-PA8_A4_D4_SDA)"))
 (segment (start 157.610366 92.024) (end 119.301 92.024) (width 0.2) (layer "B.Cu") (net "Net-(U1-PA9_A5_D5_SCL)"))
 (segment (start 167.65 83.54) (end 166.094366 83.54) (width 0.2) (layer "B.Cu") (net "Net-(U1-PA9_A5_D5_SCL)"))
 (segment (start 166.094366 83.54) (end 157.610366 92.024) (width 0.2) (layer "B.Cu") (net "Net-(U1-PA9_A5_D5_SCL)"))
 (segment (start 119.301 92.024) (end 118.2 93.125) (width 0.2) (layer "B.Cu") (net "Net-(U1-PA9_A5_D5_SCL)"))
 (segment (start 159 70.641586) (end 144.5 85.141586) (width 0.2) (layer "B.Cu") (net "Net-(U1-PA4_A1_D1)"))
 (segment (start 158 59.5) (end 159 60.5) (width 0.2) (layer "B.Cu") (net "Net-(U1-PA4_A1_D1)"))
 (segment (start 130 59.5) (end 158 59.5) (width 0.2) (layer "B.Cu") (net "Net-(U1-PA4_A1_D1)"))
 (segment (start 121.5 69) (end 130 60.5) (width 0.2) (layer "B.Cu") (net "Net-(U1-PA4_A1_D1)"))
 (segment (start 111.165 90) (end 108.04 93.125) (width 0.2) (layer "B.Cu") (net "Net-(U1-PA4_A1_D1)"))
 (segment (start 144.5 85.141586) (end 144.5 90) (width 0.2) (layer "B.Cu") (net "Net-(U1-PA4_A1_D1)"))
 (segment (start 159 60.5) (end 159 70.641586) (width 0.2) (layer "B.Cu") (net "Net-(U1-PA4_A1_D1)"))
 (segment (start 130 60.5) (end 130 59.5) (width 0.2) (layer "B.Cu") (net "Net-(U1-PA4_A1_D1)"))
 (segment (start 144.5 90) (end 111.165 90) (width 0.2) (layer "B.Cu") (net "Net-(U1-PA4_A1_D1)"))
 (segment (start 159.5 70.708686) (end 145 85.208686) (width 0.2) (layer "B.Cu") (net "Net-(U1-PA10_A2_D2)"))
 (segment (start 107 69) (end 119 69) (width 0.2) (layer "B.Cu") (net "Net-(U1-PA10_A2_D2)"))
 (segment (start 145 85.208686) (end 145 90.5) (width 0.2) (layer "B.Cu") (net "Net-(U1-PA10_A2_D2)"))
 (segment (start 113.205 90.5) (end 110.58 93.125) (width 0.2) (layer "B.Cu") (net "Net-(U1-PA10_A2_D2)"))
 (segment (start 145 90.5) (end 113.205 90.5) (width 0.2) (layer "B.Cu") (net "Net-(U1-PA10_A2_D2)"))
 (segment (start 128 59) (end 158.5 59) (width 0.2) (layer "B.Cu") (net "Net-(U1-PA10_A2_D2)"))
 (segment (start 119 69) (end 128 60) (width 0.2) (layer "B.Cu") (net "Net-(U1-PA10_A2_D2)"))
 (segment (start 128 60) (end 128 59) (width 0.2) (layer "B.Cu") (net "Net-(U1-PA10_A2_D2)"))
 (segment (start 158.5 59) (end 159.5 60) (width 0.2) (layer "B.Cu") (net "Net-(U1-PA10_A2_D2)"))
 (segment (start 159.5 60) (end 159.5 70.708686) (width 0.2) (layer "B.Cu") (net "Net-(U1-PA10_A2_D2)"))
 (segment (start 106.461108 70.301) (end 122.038892 70.301) (width 0.2) (layer "B.Cu") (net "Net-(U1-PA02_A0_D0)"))
 (segment (start 107 64) (end 105.699 65.301) (width 0.2) (layer "B.Cu") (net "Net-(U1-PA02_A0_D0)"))
 (segment (start 105.699 69.538892) (end 106.461108 70.301) (width 0.2) (layer "B.Cu") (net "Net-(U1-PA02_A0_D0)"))
 (segment (start 144 89.5) (end 111 89.5) (width 0.2) (layer "B.Cu") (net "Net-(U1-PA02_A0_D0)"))
 (segment (start 106.625 92) (end 105.5 93.125) (width 0.2) (layer "B.Cu") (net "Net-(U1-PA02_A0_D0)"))
 (segment (start 122.919946 69.419946) (end 122.919946 69.28874) (width 0.2) (layer "B.Cu") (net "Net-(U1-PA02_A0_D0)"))
 (segment (start 157.5 60.5) (end 157.5 61.4329) (width 0.2) (layer "B.Cu") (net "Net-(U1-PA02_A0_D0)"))
 (segment (start 131.708686 60.5) (end 157.5 60.5) (width 0.2) (layer "B.Cu") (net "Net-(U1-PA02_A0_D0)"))
 (segment (start 157.5 61.4329) (end 156.299 62.6339) (width 0.2) (layer "B.Cu") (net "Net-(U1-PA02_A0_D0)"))
 (segment (start 122.038892 70.301) (end 122.919946 69.419946) (width 0.2) (layer "B.Cu") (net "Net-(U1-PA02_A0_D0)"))
 (segment (start 122.919946 69.28874) (end 131.708686 60.5) (width 0.2) (layer "B.Cu") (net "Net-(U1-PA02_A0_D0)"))
 (segment (start 156.299 72.775486) (end 144 85.074486) (width 0.2) (layer "B.Cu") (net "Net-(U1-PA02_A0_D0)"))
 (segment (start 111 89.5) (end 108.5 92) (width 0.2) (layer "B.Cu") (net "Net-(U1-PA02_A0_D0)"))
 (segment (start 156.299 62.6339) (end 156.299 72.775486) (width 0.2) (layer "B.Cu") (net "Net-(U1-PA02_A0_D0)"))
 (segment (start 144 85.074486) (end 144 89.5) (width 0.2) (layer "B.Cu") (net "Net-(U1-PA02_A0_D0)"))
 (segment (start 105.699 65.301) (end 105.699 69.538892) (width 0.2) (layer "B.Cu") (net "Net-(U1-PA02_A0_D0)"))
 (segment (start 108.5 92) (end 106.625 92) (width 0.2) (layer "B.Cu") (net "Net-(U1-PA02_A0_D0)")))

